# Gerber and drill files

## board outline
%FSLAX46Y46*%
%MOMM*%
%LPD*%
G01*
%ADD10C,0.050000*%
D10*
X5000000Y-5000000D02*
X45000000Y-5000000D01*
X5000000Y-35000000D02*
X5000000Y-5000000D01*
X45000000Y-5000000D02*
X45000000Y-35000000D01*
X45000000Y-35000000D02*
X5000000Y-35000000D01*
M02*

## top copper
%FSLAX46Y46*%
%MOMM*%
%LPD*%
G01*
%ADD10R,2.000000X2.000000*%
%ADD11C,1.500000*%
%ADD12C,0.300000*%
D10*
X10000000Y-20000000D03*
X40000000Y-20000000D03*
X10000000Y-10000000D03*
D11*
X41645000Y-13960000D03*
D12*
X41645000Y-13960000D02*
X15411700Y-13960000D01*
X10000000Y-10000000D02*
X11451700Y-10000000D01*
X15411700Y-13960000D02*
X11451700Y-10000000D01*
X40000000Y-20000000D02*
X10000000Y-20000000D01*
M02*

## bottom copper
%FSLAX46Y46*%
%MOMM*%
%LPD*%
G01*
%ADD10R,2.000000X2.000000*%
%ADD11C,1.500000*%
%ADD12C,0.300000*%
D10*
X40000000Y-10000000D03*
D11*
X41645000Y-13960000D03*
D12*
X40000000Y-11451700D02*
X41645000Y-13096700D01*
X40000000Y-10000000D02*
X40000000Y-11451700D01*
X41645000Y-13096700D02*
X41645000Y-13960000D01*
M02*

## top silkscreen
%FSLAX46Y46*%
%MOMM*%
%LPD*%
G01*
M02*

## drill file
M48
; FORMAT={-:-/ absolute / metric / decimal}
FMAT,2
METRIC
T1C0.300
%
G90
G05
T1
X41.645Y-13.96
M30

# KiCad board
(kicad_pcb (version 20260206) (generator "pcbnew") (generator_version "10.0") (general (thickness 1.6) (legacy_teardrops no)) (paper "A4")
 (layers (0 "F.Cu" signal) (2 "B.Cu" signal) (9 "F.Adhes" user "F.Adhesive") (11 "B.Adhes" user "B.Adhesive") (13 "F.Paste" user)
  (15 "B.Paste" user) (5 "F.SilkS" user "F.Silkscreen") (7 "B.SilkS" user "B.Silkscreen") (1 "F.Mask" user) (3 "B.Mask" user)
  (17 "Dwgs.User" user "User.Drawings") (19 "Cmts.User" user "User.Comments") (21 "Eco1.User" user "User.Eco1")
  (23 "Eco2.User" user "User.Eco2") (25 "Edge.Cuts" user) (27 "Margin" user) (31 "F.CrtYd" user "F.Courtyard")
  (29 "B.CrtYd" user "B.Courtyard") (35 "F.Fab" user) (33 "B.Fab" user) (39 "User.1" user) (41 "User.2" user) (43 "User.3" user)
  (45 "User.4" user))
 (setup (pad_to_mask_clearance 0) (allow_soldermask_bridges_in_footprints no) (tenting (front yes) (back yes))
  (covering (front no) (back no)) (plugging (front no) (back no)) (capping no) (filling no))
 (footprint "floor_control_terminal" (layer "F.Cu") (at 10 20)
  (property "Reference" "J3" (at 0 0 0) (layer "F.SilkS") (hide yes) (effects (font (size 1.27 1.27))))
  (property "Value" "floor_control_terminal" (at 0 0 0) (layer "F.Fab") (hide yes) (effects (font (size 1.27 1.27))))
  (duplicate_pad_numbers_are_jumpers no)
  (pad "1" smd rect (at 0 0) (size 2 2) (layers "F.Cu" "F.Mask" "F.Paste") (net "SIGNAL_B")))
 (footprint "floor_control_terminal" (layer "F.Cu") (at 40 20)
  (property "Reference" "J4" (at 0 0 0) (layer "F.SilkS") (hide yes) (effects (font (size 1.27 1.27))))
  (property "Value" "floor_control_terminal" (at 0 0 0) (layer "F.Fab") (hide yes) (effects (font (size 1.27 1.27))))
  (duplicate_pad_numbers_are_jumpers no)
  (pad "1" smd rect (at 0 0) (size 2 2) (layers "F.Cu" "F.Mask" "F.Paste") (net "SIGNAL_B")))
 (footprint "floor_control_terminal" (layer "F.Cu") (at 10 10)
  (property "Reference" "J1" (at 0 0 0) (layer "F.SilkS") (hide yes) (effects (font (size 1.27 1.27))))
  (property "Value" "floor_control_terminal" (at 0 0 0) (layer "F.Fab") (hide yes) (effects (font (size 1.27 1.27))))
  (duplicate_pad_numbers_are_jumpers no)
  (pad "1" smd rect (at 0 0) (size 2 2) (layers "F.Cu" "F.Mask" "F.Paste") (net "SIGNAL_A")))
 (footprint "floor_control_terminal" (layer "B.Cu") (at 40 10)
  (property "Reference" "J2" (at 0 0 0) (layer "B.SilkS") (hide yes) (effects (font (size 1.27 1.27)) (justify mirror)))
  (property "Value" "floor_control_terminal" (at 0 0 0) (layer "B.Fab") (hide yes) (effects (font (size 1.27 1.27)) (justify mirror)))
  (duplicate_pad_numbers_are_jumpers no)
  (pad "1" smd rect (at 0 0) (size 2 2) (layers "B.Cu" "B.Mask" "B.Paste") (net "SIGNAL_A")))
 (gr_line (start 5 5) (end 45 5) (stroke (width 0.05) (type default)) (layer "Edge.Cuts"))
 (gr_line (start 5 35) (end 5 5) (stroke (width 0.05) (type default)) (layer "Edge.Cuts"))
 (gr_line (start 45 5) (end 45 35) (stroke (width 0.05) (type default)) (layer "Edge.Cuts"))
 (gr_line (start 45 35) (end 5 35) (stroke (width 0.05) (type default)) (layer "Edge.Cuts"))
 (segment (start 41.645 13.96) (end 15.4117 13.96) (width 0.3) (layer "F.Cu") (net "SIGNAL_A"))
 (segment (start 10 10) (end 11.4517 10) (width 0.3) (layer "F.Cu") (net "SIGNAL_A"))
 (segment (start 15.4117 13.96) (end 11.4517 10) (width 0.3) (layer "F.Cu") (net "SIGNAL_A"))
 (via (at 41.645 13.96) (size 1.5) (drill 0.3) (layers "F.Cu" "B.Cu") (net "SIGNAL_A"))
 (segment (start 40 11.4517) (end 41.645 13.0967) (width 0.3) (layer "B.Cu") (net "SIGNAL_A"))
 (segment (start 40 10) (end 40 11.4517) (width 0.3) (layer "B.Cu") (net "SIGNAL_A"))
 (segment (start 41.645 13.0967) (end 41.645 13.96) (width 0.3) (layer "B.Cu") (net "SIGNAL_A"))
 (segment (start 40 20) (end 10 20) (width 0.3) (layer "F.Cu") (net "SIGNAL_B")))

